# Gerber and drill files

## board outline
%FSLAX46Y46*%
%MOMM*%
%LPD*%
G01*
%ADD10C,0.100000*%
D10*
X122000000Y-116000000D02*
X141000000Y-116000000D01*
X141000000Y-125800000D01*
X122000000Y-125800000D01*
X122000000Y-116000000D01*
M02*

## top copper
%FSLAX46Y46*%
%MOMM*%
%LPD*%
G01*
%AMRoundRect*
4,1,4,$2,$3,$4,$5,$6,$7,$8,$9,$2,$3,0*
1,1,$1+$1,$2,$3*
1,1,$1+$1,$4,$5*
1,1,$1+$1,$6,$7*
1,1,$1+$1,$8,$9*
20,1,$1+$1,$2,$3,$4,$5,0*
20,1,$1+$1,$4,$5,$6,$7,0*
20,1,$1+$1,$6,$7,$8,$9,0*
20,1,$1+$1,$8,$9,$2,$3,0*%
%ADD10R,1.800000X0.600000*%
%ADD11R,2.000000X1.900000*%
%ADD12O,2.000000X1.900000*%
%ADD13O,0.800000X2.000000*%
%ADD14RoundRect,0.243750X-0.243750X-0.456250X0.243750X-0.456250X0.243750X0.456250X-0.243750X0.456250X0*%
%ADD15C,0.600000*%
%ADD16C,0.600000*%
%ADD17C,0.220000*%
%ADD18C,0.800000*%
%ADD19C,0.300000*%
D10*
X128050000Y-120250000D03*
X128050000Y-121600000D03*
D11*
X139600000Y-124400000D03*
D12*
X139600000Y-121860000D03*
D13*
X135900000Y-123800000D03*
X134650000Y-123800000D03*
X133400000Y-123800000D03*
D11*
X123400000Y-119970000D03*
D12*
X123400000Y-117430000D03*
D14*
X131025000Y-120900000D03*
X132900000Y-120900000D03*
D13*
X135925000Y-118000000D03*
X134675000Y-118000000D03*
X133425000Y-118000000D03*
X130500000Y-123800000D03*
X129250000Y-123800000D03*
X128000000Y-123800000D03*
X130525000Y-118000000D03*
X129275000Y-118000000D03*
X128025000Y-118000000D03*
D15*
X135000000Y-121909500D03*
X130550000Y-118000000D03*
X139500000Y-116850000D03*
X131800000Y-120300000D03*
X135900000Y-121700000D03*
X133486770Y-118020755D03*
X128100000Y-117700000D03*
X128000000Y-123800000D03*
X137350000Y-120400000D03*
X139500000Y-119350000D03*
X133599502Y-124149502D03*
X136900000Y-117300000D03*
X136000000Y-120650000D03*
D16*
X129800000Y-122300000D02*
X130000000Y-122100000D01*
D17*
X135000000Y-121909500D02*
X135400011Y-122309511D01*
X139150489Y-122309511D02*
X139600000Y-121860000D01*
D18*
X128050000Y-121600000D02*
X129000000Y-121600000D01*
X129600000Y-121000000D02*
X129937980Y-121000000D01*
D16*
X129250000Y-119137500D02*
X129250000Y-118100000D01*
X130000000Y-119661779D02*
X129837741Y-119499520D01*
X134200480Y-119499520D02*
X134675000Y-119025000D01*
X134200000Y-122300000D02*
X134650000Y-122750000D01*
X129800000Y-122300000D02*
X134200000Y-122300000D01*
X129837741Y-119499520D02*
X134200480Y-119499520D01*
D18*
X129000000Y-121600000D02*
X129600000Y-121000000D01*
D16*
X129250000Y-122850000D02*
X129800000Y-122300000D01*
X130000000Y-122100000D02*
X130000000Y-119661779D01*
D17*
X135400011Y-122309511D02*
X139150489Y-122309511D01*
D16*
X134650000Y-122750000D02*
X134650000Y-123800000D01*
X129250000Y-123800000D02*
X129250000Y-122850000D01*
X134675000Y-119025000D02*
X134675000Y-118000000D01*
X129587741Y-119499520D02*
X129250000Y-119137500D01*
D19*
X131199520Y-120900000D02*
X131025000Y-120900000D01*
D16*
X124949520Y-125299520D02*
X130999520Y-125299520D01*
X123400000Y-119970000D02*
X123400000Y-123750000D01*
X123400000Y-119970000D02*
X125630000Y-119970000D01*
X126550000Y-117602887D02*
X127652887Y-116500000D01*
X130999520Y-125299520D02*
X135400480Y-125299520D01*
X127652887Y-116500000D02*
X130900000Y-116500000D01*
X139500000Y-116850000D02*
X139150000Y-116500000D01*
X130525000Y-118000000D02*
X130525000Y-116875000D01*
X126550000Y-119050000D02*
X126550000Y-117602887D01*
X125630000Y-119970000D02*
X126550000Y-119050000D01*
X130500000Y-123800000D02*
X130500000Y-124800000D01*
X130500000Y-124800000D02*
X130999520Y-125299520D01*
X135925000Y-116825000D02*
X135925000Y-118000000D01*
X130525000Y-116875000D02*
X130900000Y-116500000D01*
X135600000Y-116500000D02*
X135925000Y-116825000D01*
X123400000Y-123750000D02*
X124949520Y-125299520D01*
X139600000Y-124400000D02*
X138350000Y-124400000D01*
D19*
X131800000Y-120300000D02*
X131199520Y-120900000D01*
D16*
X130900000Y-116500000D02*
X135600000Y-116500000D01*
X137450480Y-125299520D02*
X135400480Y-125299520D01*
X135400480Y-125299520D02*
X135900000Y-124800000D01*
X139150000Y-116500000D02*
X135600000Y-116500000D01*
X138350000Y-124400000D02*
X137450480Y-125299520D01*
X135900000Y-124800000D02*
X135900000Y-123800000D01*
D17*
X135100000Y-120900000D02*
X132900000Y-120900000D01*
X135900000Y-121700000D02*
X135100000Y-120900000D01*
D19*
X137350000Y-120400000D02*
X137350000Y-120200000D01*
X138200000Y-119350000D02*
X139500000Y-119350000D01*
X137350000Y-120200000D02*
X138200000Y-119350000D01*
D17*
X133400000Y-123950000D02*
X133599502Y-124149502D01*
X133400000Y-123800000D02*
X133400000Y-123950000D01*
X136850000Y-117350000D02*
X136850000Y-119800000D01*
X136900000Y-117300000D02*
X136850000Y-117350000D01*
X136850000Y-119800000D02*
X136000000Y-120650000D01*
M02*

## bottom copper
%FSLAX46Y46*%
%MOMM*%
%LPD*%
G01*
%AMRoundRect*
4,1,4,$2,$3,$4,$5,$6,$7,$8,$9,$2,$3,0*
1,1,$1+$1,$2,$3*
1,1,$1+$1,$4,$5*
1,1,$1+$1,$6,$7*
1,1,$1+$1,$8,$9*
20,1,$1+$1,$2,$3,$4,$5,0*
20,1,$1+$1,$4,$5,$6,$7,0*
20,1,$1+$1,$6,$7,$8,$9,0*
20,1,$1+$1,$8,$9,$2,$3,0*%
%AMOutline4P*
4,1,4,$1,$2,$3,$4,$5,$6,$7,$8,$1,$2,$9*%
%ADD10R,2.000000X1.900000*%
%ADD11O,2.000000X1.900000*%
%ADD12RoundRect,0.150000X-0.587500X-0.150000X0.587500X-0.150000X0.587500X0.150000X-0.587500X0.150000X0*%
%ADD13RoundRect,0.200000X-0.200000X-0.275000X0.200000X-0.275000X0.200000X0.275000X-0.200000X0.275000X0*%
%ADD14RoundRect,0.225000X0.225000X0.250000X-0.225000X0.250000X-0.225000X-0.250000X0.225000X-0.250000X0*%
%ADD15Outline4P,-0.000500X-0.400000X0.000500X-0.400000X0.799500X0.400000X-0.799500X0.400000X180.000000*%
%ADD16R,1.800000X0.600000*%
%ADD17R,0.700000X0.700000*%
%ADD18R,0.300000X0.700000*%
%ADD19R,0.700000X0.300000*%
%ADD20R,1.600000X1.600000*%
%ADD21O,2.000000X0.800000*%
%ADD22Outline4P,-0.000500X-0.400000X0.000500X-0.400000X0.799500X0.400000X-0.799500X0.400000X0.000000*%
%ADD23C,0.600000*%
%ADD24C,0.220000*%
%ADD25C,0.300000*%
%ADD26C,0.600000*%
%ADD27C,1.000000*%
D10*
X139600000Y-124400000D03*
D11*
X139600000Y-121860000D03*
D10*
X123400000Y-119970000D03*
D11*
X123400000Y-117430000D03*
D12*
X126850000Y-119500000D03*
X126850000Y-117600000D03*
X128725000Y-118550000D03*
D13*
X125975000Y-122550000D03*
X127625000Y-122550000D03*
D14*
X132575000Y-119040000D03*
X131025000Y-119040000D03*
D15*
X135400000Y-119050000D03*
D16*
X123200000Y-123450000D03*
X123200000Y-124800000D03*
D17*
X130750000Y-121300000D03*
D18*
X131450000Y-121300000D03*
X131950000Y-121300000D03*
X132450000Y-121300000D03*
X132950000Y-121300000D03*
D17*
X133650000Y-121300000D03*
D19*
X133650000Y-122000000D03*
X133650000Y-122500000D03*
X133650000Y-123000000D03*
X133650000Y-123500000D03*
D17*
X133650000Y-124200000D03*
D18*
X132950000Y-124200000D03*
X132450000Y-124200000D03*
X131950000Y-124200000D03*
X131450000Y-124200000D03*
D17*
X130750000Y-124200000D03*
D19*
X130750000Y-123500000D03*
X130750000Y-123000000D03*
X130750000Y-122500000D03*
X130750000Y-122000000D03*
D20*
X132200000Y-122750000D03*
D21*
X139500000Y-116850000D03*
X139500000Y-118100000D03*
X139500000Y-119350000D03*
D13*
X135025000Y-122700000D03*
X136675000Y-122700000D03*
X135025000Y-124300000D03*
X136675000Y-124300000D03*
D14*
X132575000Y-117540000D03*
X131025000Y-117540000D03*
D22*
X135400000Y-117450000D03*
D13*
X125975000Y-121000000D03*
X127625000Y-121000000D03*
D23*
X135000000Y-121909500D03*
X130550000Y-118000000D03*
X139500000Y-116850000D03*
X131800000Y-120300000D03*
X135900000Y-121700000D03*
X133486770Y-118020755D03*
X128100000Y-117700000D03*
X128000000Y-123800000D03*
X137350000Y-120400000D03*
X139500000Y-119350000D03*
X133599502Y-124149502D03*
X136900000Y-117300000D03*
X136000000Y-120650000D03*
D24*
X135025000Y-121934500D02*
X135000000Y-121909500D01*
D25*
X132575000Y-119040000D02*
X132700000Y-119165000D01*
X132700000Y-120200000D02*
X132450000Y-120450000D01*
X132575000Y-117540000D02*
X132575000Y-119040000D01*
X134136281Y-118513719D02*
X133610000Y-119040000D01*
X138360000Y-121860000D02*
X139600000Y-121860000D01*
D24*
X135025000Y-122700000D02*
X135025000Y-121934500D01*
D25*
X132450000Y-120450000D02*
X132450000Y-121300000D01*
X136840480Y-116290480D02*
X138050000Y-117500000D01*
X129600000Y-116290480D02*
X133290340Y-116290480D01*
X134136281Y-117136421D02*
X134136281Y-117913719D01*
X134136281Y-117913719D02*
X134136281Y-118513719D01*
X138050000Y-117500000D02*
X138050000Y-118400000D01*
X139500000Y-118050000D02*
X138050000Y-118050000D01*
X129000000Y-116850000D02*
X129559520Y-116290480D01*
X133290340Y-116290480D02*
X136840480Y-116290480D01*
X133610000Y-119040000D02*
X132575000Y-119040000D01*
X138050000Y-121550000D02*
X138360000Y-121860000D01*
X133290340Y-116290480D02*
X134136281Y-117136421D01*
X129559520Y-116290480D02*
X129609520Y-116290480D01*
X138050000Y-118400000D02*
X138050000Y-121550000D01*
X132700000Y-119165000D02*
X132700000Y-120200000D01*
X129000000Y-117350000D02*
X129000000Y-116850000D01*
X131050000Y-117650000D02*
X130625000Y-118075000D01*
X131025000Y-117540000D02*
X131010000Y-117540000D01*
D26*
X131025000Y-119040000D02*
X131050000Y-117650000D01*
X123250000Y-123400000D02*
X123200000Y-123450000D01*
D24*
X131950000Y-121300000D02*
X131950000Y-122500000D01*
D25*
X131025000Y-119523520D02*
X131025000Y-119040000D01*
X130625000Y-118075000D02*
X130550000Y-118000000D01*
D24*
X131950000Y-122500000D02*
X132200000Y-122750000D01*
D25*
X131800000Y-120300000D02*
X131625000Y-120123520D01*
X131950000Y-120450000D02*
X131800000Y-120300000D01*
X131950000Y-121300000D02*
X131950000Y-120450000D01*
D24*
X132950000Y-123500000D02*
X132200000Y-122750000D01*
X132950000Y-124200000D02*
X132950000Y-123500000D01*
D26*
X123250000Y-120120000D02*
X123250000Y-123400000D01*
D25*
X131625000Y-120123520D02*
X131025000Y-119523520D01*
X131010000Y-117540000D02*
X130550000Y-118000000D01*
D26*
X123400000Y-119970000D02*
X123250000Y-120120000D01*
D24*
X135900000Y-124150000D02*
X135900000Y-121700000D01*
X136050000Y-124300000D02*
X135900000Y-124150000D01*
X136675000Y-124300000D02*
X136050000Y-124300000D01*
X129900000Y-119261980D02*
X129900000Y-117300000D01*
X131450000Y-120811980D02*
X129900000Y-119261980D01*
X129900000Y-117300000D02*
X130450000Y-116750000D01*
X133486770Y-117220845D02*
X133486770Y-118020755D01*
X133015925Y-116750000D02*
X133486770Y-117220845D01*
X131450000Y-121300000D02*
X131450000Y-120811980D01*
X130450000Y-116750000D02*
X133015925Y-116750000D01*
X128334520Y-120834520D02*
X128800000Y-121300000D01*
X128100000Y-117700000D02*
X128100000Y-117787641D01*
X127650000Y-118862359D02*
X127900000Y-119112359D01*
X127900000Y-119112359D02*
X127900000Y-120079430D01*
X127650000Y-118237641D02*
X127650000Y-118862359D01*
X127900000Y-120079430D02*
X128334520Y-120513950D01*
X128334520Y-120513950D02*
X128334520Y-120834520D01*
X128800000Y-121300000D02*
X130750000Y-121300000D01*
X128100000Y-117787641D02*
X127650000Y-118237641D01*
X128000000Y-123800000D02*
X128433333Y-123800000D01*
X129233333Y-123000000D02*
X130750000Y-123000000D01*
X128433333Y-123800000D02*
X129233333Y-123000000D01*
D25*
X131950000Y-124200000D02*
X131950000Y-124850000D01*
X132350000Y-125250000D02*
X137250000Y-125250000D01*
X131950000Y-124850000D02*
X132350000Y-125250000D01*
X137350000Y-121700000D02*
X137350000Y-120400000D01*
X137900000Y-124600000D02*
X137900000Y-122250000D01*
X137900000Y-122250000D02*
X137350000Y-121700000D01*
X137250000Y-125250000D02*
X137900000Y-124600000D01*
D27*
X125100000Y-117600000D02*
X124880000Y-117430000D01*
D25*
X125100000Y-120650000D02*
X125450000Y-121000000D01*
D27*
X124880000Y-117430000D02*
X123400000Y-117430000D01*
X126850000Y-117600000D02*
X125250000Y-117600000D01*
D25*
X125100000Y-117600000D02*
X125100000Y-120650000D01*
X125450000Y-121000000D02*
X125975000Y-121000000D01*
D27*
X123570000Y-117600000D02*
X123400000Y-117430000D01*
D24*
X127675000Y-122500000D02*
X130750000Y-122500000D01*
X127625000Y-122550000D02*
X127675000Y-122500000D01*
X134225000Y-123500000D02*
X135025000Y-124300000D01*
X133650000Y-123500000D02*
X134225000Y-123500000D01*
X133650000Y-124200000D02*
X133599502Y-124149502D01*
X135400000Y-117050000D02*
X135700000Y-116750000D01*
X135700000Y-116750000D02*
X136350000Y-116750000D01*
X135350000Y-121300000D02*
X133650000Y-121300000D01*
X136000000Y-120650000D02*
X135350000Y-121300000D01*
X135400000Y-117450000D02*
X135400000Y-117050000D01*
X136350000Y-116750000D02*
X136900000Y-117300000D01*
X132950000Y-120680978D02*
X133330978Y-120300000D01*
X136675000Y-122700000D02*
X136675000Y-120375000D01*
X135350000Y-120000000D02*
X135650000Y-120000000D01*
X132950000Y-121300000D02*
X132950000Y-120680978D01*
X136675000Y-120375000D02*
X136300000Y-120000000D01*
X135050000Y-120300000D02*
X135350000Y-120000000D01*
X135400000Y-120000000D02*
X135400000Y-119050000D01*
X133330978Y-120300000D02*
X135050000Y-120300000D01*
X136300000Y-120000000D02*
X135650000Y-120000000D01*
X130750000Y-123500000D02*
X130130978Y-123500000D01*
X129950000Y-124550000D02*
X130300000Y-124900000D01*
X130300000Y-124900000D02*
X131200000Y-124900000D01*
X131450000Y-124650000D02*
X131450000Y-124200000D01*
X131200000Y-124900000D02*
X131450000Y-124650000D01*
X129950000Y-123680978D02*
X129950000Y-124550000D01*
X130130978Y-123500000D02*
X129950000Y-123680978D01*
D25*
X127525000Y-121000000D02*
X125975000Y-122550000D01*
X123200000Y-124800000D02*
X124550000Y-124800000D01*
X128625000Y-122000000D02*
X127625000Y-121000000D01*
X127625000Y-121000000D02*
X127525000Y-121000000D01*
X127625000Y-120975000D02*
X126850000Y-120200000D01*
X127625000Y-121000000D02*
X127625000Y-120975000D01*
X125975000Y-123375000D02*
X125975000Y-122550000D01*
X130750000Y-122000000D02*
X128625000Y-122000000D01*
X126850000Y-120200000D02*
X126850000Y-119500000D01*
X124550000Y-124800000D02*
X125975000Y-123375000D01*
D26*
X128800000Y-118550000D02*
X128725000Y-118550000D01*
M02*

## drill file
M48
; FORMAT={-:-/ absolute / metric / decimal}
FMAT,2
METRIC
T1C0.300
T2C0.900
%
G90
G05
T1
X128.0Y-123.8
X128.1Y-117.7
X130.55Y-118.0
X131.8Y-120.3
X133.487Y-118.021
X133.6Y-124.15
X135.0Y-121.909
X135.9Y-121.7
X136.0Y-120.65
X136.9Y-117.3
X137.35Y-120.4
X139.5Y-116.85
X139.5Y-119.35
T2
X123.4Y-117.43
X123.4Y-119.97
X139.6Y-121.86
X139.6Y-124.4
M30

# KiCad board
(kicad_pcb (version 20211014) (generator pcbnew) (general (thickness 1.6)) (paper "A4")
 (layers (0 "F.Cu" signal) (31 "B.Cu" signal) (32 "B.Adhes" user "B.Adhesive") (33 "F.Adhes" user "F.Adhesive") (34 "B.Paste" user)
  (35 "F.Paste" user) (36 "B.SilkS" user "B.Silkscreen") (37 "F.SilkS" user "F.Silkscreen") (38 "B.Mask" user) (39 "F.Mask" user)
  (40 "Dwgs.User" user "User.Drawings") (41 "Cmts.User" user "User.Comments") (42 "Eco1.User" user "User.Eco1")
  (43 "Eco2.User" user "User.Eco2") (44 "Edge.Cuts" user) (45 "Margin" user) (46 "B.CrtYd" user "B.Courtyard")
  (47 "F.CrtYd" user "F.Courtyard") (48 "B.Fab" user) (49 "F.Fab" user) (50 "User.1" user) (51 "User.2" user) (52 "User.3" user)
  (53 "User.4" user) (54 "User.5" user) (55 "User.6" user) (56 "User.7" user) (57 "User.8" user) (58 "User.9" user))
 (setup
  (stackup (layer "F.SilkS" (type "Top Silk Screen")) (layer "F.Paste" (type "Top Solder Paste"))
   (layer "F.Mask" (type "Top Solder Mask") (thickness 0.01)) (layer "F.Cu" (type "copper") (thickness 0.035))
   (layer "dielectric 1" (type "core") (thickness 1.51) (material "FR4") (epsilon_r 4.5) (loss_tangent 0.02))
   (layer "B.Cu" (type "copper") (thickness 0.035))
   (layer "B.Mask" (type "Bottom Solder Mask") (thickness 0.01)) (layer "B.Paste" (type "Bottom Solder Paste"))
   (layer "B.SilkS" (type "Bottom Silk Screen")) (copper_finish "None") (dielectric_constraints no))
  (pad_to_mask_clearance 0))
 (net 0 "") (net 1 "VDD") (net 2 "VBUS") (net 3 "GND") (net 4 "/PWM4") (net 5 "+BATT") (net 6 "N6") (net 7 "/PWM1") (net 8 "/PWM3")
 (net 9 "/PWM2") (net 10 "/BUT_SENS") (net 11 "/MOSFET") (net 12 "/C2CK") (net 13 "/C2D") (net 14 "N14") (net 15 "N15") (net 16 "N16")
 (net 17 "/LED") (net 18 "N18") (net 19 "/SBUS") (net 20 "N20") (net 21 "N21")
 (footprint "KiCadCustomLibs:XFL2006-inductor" (layer "F.Cu") (at 128.05 120.925 -90)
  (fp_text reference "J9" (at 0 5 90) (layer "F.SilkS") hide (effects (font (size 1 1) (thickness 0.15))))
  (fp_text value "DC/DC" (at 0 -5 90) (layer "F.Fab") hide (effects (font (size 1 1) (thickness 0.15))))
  (pad "1" smd rect locked (at -0.675 0 270) (size 0.6 1.8) (layers "F.Cu" "F.Paste" "F.Mask") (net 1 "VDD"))
  (pad "2" smd rect locked (at 0.675 0 270) (size 0.6 1.8) (layers "F.Cu" "F.Paste" "F.Mask") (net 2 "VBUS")))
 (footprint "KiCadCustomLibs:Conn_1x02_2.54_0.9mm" (layer "F.Cu") (at 139.6 124.4 180)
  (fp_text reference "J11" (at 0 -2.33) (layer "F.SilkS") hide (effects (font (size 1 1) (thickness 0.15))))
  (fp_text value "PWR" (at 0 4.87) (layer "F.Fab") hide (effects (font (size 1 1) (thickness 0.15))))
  (pad "1" thru_hole rect locked (at 0 0 180) (size 2 1.9) (drill 0.9) (layers *.Cu *.Mask) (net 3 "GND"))
  (pad "2" thru_hole oval locked (at 0 2.54 180) (size 2 1.9) (drill 0.9) (layers *.Cu *.Mask) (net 2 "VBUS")))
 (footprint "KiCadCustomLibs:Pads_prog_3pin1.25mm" (layer "F.Cu") (at 134.675 123.8 180)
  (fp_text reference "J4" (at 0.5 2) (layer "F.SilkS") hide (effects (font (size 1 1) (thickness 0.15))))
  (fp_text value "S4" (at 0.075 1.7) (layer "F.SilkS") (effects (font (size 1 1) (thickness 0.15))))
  (pad "1" smd oval locked (at -1.225 0 180) (size 0.8 2) (layers "F.Cu" "F.Paste" "F.Mask") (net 3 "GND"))
  (pad "2" smd oval locked (at 0.025 0 180) (size 0.8 2) (layers "F.Cu" "F.Paste" "F.Mask") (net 2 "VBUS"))
  (pad "3" smd oval locked (at 1.275 0 180) (size 0.8 2) (layers "F.Cu" "F.Paste" "F.Mask") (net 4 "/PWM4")))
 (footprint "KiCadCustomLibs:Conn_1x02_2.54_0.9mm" (layer "F.Cu") (at 123.4 119.97 180)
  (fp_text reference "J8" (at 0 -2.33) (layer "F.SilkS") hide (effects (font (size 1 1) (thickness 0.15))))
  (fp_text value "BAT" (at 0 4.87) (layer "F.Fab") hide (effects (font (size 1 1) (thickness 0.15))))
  (pad "1" thru_hole rect locked (at 0 0 180) (size 2 1.9) (drill 0.9) (layers *.Cu *.Mask) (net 3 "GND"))
  (pad "2" thru_hole oval locked (at 0 2.54 180) (size 2 1.9) (drill 0.9) (layers *.Cu *.Mask) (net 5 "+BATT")))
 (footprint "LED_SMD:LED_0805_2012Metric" (layer "F.Cu") (at 131.9625 120.9)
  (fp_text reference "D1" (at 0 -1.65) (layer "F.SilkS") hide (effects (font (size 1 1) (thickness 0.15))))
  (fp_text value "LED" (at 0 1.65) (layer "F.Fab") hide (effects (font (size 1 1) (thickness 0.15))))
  (pad "1" smd roundrect (at -0.9375 0) (size 0.975 1.4) (layers "F.Cu" "F.Paste" "F.Mask") (roundrect_rratio 0.25) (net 3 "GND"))
  (pad "2" smd roundrect (at 0.9375 0) (size 0.975 1.4) (layers "F.Cu" "F.Paste" "F.Mask") (roundrect_rratio 0.25) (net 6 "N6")))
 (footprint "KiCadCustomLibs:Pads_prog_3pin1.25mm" (layer "F.Cu") (at 134.7 118 180)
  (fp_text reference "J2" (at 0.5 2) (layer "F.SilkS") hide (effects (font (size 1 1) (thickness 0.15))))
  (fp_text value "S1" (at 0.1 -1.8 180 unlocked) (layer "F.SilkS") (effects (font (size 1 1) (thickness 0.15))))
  (pad "1" smd oval locked (at -1.225 0 180) (size 0.8 2) (layers "F.Cu" "F.Paste" "F.Mask") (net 3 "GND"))
  (pad "2" smd oval locked (at 0.025 0 180) (size 0.8 2) (layers "F.Cu" "F.Paste" "F.Mask") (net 2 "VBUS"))
  (pad "3" smd oval locked (at 1.275 0 180) (size 0.8 2) (layers "F.Cu" "F.Paste" "F.Mask") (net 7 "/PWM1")))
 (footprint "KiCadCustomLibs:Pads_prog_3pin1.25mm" (layer "F.Cu") (at 129.275 123.8 180)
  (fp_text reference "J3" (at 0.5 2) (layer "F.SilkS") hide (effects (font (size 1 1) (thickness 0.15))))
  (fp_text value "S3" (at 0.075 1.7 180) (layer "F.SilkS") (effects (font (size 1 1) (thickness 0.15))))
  (pad "1" smd oval locked (at -1.225 0 180) (size 0.8 2) (layers "F.Cu" "F.Paste" "F.Mask") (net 3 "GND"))
  (pad "2" smd oval locked (at 0.025 0 180) (size 0.8 2) (layers "F.Cu" "F.Paste" "F.Mask") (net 2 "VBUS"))
  (pad "3" smd oval locked (at 1.275 0 180) (size 0.8 2) (layers "F.Cu" "F.Paste" "F.Mask") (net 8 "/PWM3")))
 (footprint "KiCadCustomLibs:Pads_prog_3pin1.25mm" (layer "F.Cu") (at 129.3 118 180)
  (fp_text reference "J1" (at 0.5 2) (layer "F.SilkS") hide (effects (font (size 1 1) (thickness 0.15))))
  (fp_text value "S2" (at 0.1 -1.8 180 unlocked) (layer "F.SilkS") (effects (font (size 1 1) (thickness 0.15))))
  (pad "1" smd oval locked (at -1.225 0 180) (size 0.8 2) (layers "F.Cu" "F.Paste" "F.Mask") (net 3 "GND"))
  (pad "2" smd oval locked (at 0.025 0 180) (size 0.8 2) (layers "F.Cu" "F.Paste" "F.Mask") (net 2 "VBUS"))
  (pad "3" smd oval locked (at 1.275 0 180) (size 0.8 2) (layers "F.Cu" "F.Paste" "F.Mask") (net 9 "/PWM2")))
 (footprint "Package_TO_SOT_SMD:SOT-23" (layer "B.Cu") (at 127.7875 118.55)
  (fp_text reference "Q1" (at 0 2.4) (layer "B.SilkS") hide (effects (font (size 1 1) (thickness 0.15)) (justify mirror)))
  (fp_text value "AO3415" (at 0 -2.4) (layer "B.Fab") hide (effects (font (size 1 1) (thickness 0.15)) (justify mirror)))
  (pad "1" smd roundrect (at -0.9375 0.95) (size 1.475 0.6) (layers "B.Cu" "B.Paste" "B.Mask") (roundrect_rratio 0.25) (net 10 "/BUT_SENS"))
  (pad "2" smd roundrect (at -0.9375 -0.95) (size 1.475 0.6) (layers "B.Cu" "B.Paste" "B.Mask") (roundrect_rratio 0.25) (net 5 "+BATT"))
  (pad "3" smd roundrect (at 0.9375 0) (size 1.475 0.6) (layers "B.Cu" "B.Paste" "B.Mask") (roundrect_rratio 0.25) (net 1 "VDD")))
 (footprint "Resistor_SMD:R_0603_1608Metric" (layer "B.Cu") (at 126.8 122.55)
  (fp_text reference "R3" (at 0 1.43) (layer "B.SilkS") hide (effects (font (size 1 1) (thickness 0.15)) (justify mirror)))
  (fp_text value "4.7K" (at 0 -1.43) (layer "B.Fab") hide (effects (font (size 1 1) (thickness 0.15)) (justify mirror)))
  (pad "1" smd roundrect (at -0.825 0) (size 0.8 0.95) (layers "B.Cu" "B.Paste" "B.Mask") (roundrect_rratio 0.25) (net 10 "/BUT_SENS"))
  (pad "2" smd roundrect (at 0.825 0) (size 0.8 0.95) (layers "B.Cu" "B.Paste" "B.Mask") (roundrect_rratio 0.25) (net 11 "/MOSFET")))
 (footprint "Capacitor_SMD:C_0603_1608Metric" (layer "B.Cu") (at 131.8 119.04 180)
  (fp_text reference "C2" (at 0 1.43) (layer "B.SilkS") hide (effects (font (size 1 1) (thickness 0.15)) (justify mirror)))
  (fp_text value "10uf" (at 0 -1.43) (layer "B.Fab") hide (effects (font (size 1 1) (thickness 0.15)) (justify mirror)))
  (pad "1" smd roundrect (at -0.775 0 180) (size 0.9 0.95) (layers "B.Cu" "B.Paste" "B.Mask") (roundrect_rratio 0.25) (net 2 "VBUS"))
  (pad "2" smd roundrect (at 0.775 0 180) (size 0.9 0.95) (layers "B.Cu" "B.Paste" "B.Mask") (roundrect_rratio 0.25) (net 3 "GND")))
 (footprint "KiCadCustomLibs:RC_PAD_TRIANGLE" (layer "B.Cu") (at 135.4 119.05 180)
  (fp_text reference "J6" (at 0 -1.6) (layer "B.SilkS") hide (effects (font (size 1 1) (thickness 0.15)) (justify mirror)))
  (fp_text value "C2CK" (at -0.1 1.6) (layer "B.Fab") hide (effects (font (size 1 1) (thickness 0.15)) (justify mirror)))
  (pad "1" smd trapezoid locked (at 0 0 180) (size 0.8 0.8) (rect_delta 0 -0.799) (layers "B.Cu" "B.Paste" "B.Mask") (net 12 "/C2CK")))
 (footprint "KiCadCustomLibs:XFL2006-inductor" (layer "B.Cu") (at 123.2 124.125 -90)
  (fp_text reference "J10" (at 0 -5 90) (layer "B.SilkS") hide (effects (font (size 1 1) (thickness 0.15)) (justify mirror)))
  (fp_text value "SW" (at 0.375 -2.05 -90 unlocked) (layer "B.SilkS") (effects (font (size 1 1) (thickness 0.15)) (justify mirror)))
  (pad "1" smd rect locked (at -0.675 0 270) (size 0.6 1.8) (layers "B.Cu" "B.Paste" "B.Mask") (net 3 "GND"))
  (pad "2" smd rect locked (at 0.675 0 270) (size 0.6 1.8) (layers "B.Cu" "B.Paste" "B.Mask") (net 10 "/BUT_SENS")))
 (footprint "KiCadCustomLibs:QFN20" (layer "B.Cu") (at 132.2 122.75)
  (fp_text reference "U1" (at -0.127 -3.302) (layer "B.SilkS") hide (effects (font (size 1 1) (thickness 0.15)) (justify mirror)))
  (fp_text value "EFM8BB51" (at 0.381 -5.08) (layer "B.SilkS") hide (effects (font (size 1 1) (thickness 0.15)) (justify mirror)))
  (pad "1" smd rect locked (at -1.45 -1.45) (size 0.7 0.7) (layers "B.Cu" "B.Paste" "B.Mask") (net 9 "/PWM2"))
  (pad "2" smd rect locked (at -0.75 -1.45) (size 0.3 0.7) (layers "B.Cu" "B.Paste" "B.Mask") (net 7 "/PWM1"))
  (pad "3" smd rect locked (at -0.25 -1.45) (size 0.3 0.7) (layers "B.Cu" "B.Paste" "B.Mask") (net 3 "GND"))
  (pad "4" smd rect locked (at 0.25 -1.45) (size 0.3 0.7) (layers "B.Cu" "B.Paste" "B.Mask") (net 2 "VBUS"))
  (pad "5" smd rect locked (at 0.75 -1.45) (size 0.3 0.7) (layers "B.Cu" "B.Paste" "B.Mask") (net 12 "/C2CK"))
  (pad "6" smd rect locked (at 1.45 -1.45) (size 0.7 0.7) (layers "B.Cu" "B.Paste" "B.Mask") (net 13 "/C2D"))
  (pad "7" smd rect locked (at 1.45 -0.75 270) (size 0.3 0.7) (layers "B.Cu" "B.Paste" "B.Mask") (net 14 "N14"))
  (pad "8" smd rect locked (at 1.45 -0.25 270) (size 0.3 0.7) (layers "B.Cu" "B.Paste" "B.Mask") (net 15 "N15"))
  (pad "9" smd rect locked (at 1.45 0.25 270) (size 0.3 0.7) (layers "B.Cu" "B.Paste" "B.Mask") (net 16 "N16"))
  (pad "10" smd rect locked (at 1.45 0.75 270) (size 0.3 0.7) (layers "B.Cu" "B.Paste" "B.Mask") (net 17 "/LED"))
  (pad "11" smd rect locked (at 1.45 1.45) (size 0.7 0.7) (layers "B.Cu" "B.Paste" "B.Mask") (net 4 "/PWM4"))
  (pad "12" smd rect locked (at 0.75 1.45) (size 0.3 0.7) (layers "B.Cu" "B.Paste" "B.Mask") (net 3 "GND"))
  (pad "13" smd rect locked (at 0.25 1.45) (size 0.3 0.7) (layers "B.Cu" "B.Paste" "B.Mask") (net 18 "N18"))
  (pad "14" smd rect locked (at -0.25 1.45) (size 0.3 0.7) (layers "B.Cu" "B.Paste" "B.Mask") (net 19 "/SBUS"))
  (pad "15" smd rect locked (at -0.75 1.45) (size 0.3 0.7) (layers "B.Cu" "B.Paste" "B.Mask") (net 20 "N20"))
  (pad "16" smd rect locked (at -1.45 1.45) (size 0.7 0.7) (layers "B.Cu" "B.Paste" "B.Mask") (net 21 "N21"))
  (pad "17" smd rect locked (at -1.45 0.75 270) (size 0.3 0.7) (layers "B.Cu" "B.Paste" "B.Mask") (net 20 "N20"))
  (pad "18" smd rect locked (at -1.45 0.25 270) (size 0.3 0.7) (layers "B.Cu" "B.Paste" "B.Mask") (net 8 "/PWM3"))
  (pad "19" smd rect locked (at -1.45 -0.25 270) (size 0.3 0.7) (layers "B.Cu" "B.Paste" "B.Mask") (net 11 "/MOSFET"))
  (pad "20" smd rect locked (at -1.45 -0.75 270) (size 0.3 0.7) (layers "B.Cu" "B.Paste" "B.Mask") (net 10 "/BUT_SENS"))
  (pad "21" smd rect locked (at 0 0) (size 1.6 1.6) (layers "B.Cu" "B.Paste" "B.Mask") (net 3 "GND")))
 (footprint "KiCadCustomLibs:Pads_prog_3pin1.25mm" (layer "B.Cu") (at 139.5 118.075 -90)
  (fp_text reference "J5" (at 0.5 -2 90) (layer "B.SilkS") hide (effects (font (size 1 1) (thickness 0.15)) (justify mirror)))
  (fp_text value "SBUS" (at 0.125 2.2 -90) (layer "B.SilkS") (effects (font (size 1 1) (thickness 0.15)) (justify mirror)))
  (pad "1" smd oval locked (at -1.225 0 270) (size 0.8 2) (layers "B.Cu" "B.Paste" "B.Mask") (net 3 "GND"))
  (pad "2" smd oval locked (at 0.025 0 270) (size 0.8 2) (layers "B.Cu" "B.Paste" "B.Mask") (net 2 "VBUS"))
  (pad "3" smd oval locked (at 1.275 0 270) (size 0.8 2) (layers "B.Cu" "B.Paste" "B.Mask") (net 19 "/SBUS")))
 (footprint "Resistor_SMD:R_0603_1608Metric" (layer "B.Cu") (at 135.85 122.7)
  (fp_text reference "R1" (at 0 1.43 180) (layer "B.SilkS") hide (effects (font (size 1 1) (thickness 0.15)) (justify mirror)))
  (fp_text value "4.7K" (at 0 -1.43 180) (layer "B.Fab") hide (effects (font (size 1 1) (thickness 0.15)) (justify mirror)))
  (pad "1" smd roundrect (at -0.825 0) (size 0.8 0.95) (layers "B.Cu" "B.Paste" "B.Mask") (roundrect_rratio 0.25) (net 2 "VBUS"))
  (pad "2" smd roundrect (at 0.825 0) (size 0.8 0.95) (layers "B.Cu" "B.Paste" "B.Mask") (roundrect_rratio 0.25) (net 12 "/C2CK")))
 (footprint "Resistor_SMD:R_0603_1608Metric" (layer "B.Cu") (at 135.85 124.3)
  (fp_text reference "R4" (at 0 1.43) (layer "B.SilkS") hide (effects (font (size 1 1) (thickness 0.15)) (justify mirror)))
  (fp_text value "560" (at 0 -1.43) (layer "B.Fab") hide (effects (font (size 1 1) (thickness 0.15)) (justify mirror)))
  (pad "1" smd roundrect (at -0.825 0) (size 0.8 0.95) (layers "B.Cu" "B.Paste" "B.Mask") (roundrect_rratio 0.25) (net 17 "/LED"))
  (pad "2" smd roundrect (at 0.825 0) (size 0.8 0.95) (layers "B.Cu" "B.Paste" "B.Mask") (roundrect_rratio 0.25) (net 6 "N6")))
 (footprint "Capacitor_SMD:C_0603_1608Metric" (layer "B.Cu") (at 131.8 117.54 180)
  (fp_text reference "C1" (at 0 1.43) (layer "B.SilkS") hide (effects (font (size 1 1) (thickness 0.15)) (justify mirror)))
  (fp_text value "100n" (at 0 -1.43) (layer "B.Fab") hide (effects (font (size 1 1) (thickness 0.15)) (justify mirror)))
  (pad "1" smd roundrect (at -0.775 0 180) (size 0.9 0.95) (layers "B.Cu" "B.Paste" "B.Mask") (roundrect_rratio 0.25) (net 2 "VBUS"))
  (pad "2" smd roundrect (at 0.775 0 180) (size 0.9 0.95) (layers "B.Cu" "B.Paste" "B.Mask") (roundrect_rratio 0.25) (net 3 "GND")))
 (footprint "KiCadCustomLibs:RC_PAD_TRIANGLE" (layer "B.Cu") (at 135.4 117.45)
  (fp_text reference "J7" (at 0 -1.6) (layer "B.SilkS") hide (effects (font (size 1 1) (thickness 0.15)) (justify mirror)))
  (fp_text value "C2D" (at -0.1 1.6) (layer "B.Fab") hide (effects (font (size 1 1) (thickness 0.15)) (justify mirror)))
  (pad "1" smd trapezoid locked (at 0 0) (size 0.8 0.8) (rect_delta 0 -0.799) (layers "B.Cu" "B.Paste" "B.Mask") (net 13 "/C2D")))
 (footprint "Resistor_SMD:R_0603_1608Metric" (layer "B.Cu") (at 126.8 121)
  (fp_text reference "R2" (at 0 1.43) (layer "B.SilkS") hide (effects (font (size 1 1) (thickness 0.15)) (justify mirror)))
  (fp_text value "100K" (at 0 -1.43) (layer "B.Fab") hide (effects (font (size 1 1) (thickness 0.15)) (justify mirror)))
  (pad "1" smd roundrect (at -0.825 0) (size 0.8 0.95) (layers "B.Cu" "B.Paste" "B.Mask") (roundrect_rratio 0.25) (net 5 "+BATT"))
  (pad "2" smd roundrect (at 0.825 0) (size 0.8 0.95) (layers "B.Cu" "B.Paste" "B.Mask") (roundrect_rratio 0.25) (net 10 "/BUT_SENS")))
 (gr_rect (start 122 116) (end 141 125.8) (layer "Edge.Cuts") (width 0.1) (fill none))
 (segment (start 129.8 122.3) (end 130 122.1) (width 0.6) (layer "F.Cu") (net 2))
 (segment (start 135 121.9095) (end 135.400011 122.309511) (width 0.22) (layer "F.Cu") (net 2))
 (segment (start 139.150489 122.309511) (end 139.6 121.86) (width 0.22) (layer "F.Cu") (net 2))
 (segment (start 128.05 121.6) (end 129 121.6) (width 0.8) (layer "F.Cu") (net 2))
 (segment (start 129.6 121) (end 129.93798 121) (width 0.8) (layer "F.Cu") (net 2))
 (segment (start 129.25 119.1375) (end 129.25 118.1) (width 0.6) (layer "F.Cu") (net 2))
 (segment (start 130 119.661779) (end 129.837741 119.49952) (width 0.6) (layer "F.Cu") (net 2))
 (segment (start 134.20048 119.49952) (end 134.675 119.025) (width 0.6) (layer "F.Cu") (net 2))
 (segment (start 134.2 122.3) (end 134.65 122.75) (width 0.6) (layer "F.Cu") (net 2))
 (segment (start 129.8 122.3) (end 134.2 122.3) (width 0.6) (layer "F.Cu") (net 2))
 (segment (start 129.837741 119.49952) (end 134.20048 119.49952) (width 0.6) (layer "F.Cu") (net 2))
 (segment (start 129 121.6) (end 129.6 121) (width 0.8) (layer "F.Cu") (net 2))
 (segment (start 129.25 122.85) (end 129.8 122.3) (width 0.6) (layer "F.Cu") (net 2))
 (segment (start 130 122.1) (end 130 119.661779) (width 0.6) (layer "F.Cu") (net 2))
 (segment (start 135.400011 122.309511) (end 139.150489 122.309511) (width 0.22) (layer "F.Cu") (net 2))
 (segment (start 134.65 122.75) (end 134.65 123.8) (width 0.6) (layer "F.Cu") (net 2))
 (segment (start 129.25 123.8) (end 129.25 122.85) (width 0.6) (layer "F.Cu") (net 2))
 (segment (start 134.675 119.025) (end 134.675 118) (width 0.6) (layer "F.Cu") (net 2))
 (segment (start 129.587741 119.49952) (end 129.25 119.1375) (width 0.6) (layer "F.Cu") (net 2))
 (via (at 135 121.9095) (size 0.6) (drill 0.3) (layers "F.Cu" "B.Cu") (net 2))
 (segment (start 135.025 121.9345) (end 135 121.9095) (width 0.22) (layer "B.Cu") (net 2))
 (segment (start 132.575 119.04) (end 132.7 119.165) (width 0.3) (layer "B.Cu") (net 2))
 (segment (start 132.7 120.2) (end 132.45 120.45) (width 0.3) (layer "B.Cu") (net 2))
 (segment (start 132.575 117.54) (end 132.575 119.04) (width 0.3) (layer "B.Cu") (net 2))
 (segment (start 134.136281 118.513719) (end 133.61 119.04) (width 0.3) (layer "B.Cu") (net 2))
 (segment (start 138.36 121.86) (end 139.6 121.86) (width 0.3) (layer "B.Cu") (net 2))
 (segment (start 135.025 122.7) (end 135.025 121.9345) (width 0.22) (layer "B.Cu") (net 2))
 (segment (start 132.45 120.45) (end 132.45 121.3) (width 0.3) (layer "B.Cu") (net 2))
 (segment (start 136.84048 116.29048) (end 138.05 117.5) (width 0.3) (layer "B.Cu") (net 2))
 (segment (start 129.6 116.29048) (end 133.29034 116.29048) (width 0.3) (layer "B.Cu") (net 2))
 (segment (start 134.136281 117.136421) (end 134.136281 117.913719) (width 0.3) (layer "B.Cu") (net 2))
 (segment (start 134.136281 117.913719) (end 134.136281 118.513719) (width 0.3) (layer "B.Cu") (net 2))
 (segment (start 138.05 117.5) (end 138.05 118.4) (width 0.3) (layer "B.Cu") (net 2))
 (segment (start 139.5 118.05) (end 138.05 118.05) (width 0.3) (layer "B.Cu") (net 2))
 (segment (start 129 116.85) (end 129.55952 116.29048) (width 0.3) (layer "B.Cu") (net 2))
 (segment (start 133.29034 116.29048) (end 136.84048 116.29048) (width 0.3) (layer "B.Cu") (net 2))
 (segment (start 133.61 119.04) (end 132.575 119.04) (width 0.3) (layer "B.Cu") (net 2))
 (segment (start 138.05 121.55) (end 138.36 121.86) (width 0.3) (layer "B.Cu") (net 2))
 (segment (start 133.29034 116.29048) (end 134.136281 117.136421) (width 0.3) (layer "B.Cu") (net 2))
 (segment (start 129.55952 116.29048) (end 129.60952 116.29048) (width 0.3) (layer "B.Cu") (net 2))
 (segment (start 138.05 118.4) (end 138.05 121.55) (width 0.3) (layer "B.Cu") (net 2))
 (segment (start 132.7 119.165) (end 132.7 120.2) (width 0.3) (layer "B.Cu") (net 2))
 (segment (start 129 117.35) (end 129 116.85) (width 0.3) (layer "B.Cu") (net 2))
 (segment (start 131.19952 120.9) (end 131.025 120.9) (width 0.3) (layer "F.Cu") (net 3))
 (segment (start 124.94952 125.29952) (end 130.99952 125.29952) (width 0.6) (layer "F.Cu") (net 3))
 (segment (start 123.4 119.97) (end 123.4 123.75) (width 0.6) (layer "F.Cu") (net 3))
 (segment (start 123.4 119.97) (end 125.63 119.97) (width 0.6) (layer "F.Cu") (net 3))
 (segment (start 126.55 117.602887) (end 127.652887 116.5) (width 0.6) (layer "F.Cu") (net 3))
 (segment (start 130.99952 125.29952) (end 135.40048 125.29952) (width 0.6) (layer "F.Cu") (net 3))
 (segment (start 127.652887 116.5) (end 130.9 116.5) (width 0.6) (layer "F.Cu") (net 3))
 (segment (start 139.5 116.85) (end 139.15 116.5) (width 0.6) (layer "F.Cu") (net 3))
 (segment (start 130.525 118) (end 130.525 116.875) (width 0.6) (layer "F.Cu") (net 3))
 (segment (start 126.55 119.05) (end 126.55 117.602887) (width 0.6) (layer "F.Cu") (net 3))
 (segment (start 125.63 119.97) (end 126.55 119.05) (width 0.6) (layer "F.Cu") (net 3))
 (segment (start 130.5 123.8) (end 130.5 124.8) (width 0.6) (layer "F.Cu") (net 3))
 (segment (start 130.5 124.8) (end 130.99952 125.29952) (width 0.6) (layer "F.Cu") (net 3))
 (segment (start 135.925 116.825) (end 135.925 118) (width 0.6) (layer "F.Cu") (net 3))
 (segment (start 130.525 116.875) (end 130.9 116.5) (width 0.6) (layer "F.Cu") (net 3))
 (segment (start 135.6 116.5) (end 135.925 116.825) (width 0.6) (layer "F.Cu") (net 3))
 (segment (start 123.4 123.75) (end 124.94952 125.29952) (width 0.6) (layer "F.Cu") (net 3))
 (segment (start 139.6 124.4) (end 138.35 124.4) (width 0.6) (layer "F.Cu") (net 3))
 (segment (start 131.8 120.3) (end 131.19952 120.9) (width 0.3) (layer "F.Cu") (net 3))
 (segment (start 130.9 116.5) (end 135.6 116.5) (width 0.6) (layer "F.Cu") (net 3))
 (segment (start 137.45048 125.29952) (end 135.40048 125.29952) (width 0.6) (layer "F.Cu") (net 3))
 (segment (start 135.40048 125.29952) (end 135.9 124.8) (width 0.6) (layer "F.Cu") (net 3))
 (segment (start 139.15 116.5) (end 135.6 116.5) (width 0.6) (layer "F.Cu") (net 3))
 (segment (start 138.35 124.4) (end 137.45048 125.29952) (width 0.6) (layer "F.Cu") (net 3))
 (segment (start 135.9 124.8) (end 135.9 123.8) (width 0.6) (layer "F.Cu") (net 3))
 (via (at 130.55 118) (size 0.6) (drill 0.3) (layers "F.Cu" "B.Cu") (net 3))
 (via (at 139.5 116.85) (size 0.6) (drill 0.3) (layers "F.Cu" "B.Cu") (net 3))
 (via (at 131.8 120.3) (size 0.6) (drill 0.3) (layers "F.Cu" "B.Cu") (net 3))
 (segment (start 131.05 117.65) (end 130.625 118.075) (width 0.3) (layer "B.Cu") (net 3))
 (segment (start 131.025 117.54) (end 131.01 117.54) (width 0.3) (layer "B.Cu") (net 3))
 (segment (start 131.025 119.04) (end 131.05 117.65) (width 0.6) (layer "B.Cu") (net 3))
 (segment (start 123.25 123.4) (end 123.2 123.45) (width 0.6) (layer "B.Cu") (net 3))
 (segment (start 131.95 121.3) (end 131.95 122.5) (width 0.22) (layer "B.Cu") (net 3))
 (segment (start 131.025 119.52352) (end 131.025 119.04) (width 0.3) (layer "B.Cu") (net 3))
 (segment (start 130.625 118.075) (end 130.55 118) (width 0.3) (layer "B.Cu") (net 3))
 (segment (start 131.95 122.5) (end 132.2 122.75) (width 0.22) (layer "B.Cu") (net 3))
 (segment (start 131.8 120.3) (end 131.625 120.12352) (width 0.3) (layer "B.Cu") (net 3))
 (segment (start 131.95 120.45) (end 131.8 120.3) (width 0.3) (layer "B.Cu") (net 3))
 (segment (start 131.95 121.3) (end 131.95 120.45) (width 0.3) (layer "B.Cu") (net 3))
 (segment (start 132.95 123.5) (end 132.2 122.75) (width 0.22) (layer "B.Cu") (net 3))
 (segment (start 132.95 124.2) (end 132.95 123.5) (width 0.22) (layer "B.Cu") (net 3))
 (segment (start 123.25 120.12) (end 123.25 123.4) (width 0.6) (layer "B.Cu") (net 3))
 (segment (start 131.625 120.12352) (end 131.025 119.52352) (width 0.3) (layer "B.Cu") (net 3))
 (segment (start 131.01 117.54) (end 130.55 118) (width 0.3) (layer "B.Cu") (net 3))
 (segment (start 123.4 119.97) (end 123.25 120.12) (width 0.6) (layer "B.Cu") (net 3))
 (segment (start 135.1 120.9) (end 132.9 120.9) (width 0.22) (layer "F.Cu") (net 6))
 (segment (start 135.9 121.7) (end 135.1 120.9) (width 0.22) (layer "F.Cu") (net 6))
 (via (at 135.9 121.7) (size 0.6) (drill 0.3) (layers "F.Cu" "B.Cu") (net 6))
 (segment (start 135.9 124.15) (end 135.9 121.7) (width 0.22) (layer "B.Cu") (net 6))
 (segment (start 136.05 124.3) (end 135.9 124.15) (width 0.22) (layer "B.Cu") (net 6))
 (segment (start 136.675 124.3) (end 136.05 124.3) (width 0.22) (layer "B.Cu") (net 6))
 (via (at 133.48677 118.020755) (size 0.6) (drill 0.3) (layers "F.Cu" "B.Cu") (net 7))
 (segment (start 129.9 119.26198) (end 129.9 117.3) (width 0.22) (layer "B.Cu") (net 7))
 (segment (start 131.45 120.81198) (end 129.9 119.26198) (width 0.22) (layer "B.Cu") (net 7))
 (segment (start 129.9 117.3) (end 130.45 116.75) (width 0.22) (layer "B.Cu") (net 7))
 (segment (start 133.48677 117.220845) (end 133.48677 118.020755) (width 0.22) (layer "B.Cu") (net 7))
 (segment (start 133.015925 116.75) (end 133.48677 117.220845) (width 0.22) (layer "B.Cu") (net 7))
 (segment (start 131.45 121.3) (end 131.45 120.81198) (width 0.22) (layer "B.Cu") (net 7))
 (segment (start 130.45 116.75) (end 133.015925 116.75) (width 0.22) (layer "B.Cu") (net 7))
 (via (at 128.1 117.7) (size 0.6) (drill 0.3) (layers "F.Cu" "B.Cu") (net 9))
 (segment (start 128.33452 120.83452) (end 128.8 121.3) (width 0.22) (layer "B.Cu") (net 9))
 (segment (start 128.1 117.7) (end 128.1 117.787641) (width 0.22) (layer "B.Cu") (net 9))
 (segment (start 127.65 118.862359) (end 127.9 119.112359) (width 0.22) (layer "B.Cu") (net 9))
 (segment (start 127.9 119.112359) (end 127.9 120.07943) (width 0.22) (layer "B.Cu") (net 9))
 (segment (start 127.65 118.237641) (end 127.65 118.862359) (width 0.22) (layer "B.Cu") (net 9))
 (segment (start 127.9 120.07943) (end 128.33452 120.51395) (width 0.22) (layer "B.Cu") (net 9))
 (segment (start 128.33452 120.51395) (end 128.33452 120.83452) (width 0.22) (layer "B.Cu") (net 9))
 (segment (start 128.8 121.3) (end 130.75 121.3) (width 0.22) (layer "B.Cu") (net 9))
 (segment (start 128.1 117.787641) (end 127.65 118.237641) (width 0.22) (layer "B.Cu") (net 9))
 (via (at 128 123.8) (size 0.6) (drill 0.3) (layers "F.Cu" "B.Cu") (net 8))
 (segment (start 128 123.8) (end 128.433333 123.8) (width 0.22) (layer "B.Cu") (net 8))
 (segment (start 129.233333 123) (end 130.75 123) (width 0.22) (layer "B.Cu") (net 8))
 (segment (start 128.433333 123.8) (end 129.233333 123) (width 0.22) (layer "B.Cu") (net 8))
 (segment (start 137.35 120.4) (end 137.35 120.2) (width 0.3) (layer "F.Cu") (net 19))
 (segment (start 138.2 119.35) (end 139.5 119.35) (width 0.3) (layer "F.Cu") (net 19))
 (segment (start 137.35 120.2) (end 138.2 119.35) (width 0.3) (layer "F.Cu") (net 19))
 (via (at 137.35 120.4) (size 0.6) (drill 0.3) (layers "F.Cu" "B.Cu") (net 19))
 (via (at 139.5 119.35) (size 0.6) (drill 0.3) (layers "F.Cu" "B.Cu") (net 19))
 (segment (start 131.95 124.2) (end 131.95 124.85) (width 0.3) (layer "B.Cu") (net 19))
 (segment (start 132.35 125.25) (end 137.25 125.25) (width 0.3) (layer "B.Cu") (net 19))
 (segment (start 131.95 124.85) (end 132.35 125.25) (width 0.3) (layer "B.Cu") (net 19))
 (segment (start 137.35 121.7) (end 137.35 120.4) (width 0.3) (layer "B.Cu") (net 19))
 (segment (start 137.9 124.6) (end 137.9 122.25) (width 0.3) (layer "B.Cu") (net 19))
 (segment (start 137.9 122.25) (end 137.35 121.7) (width 0.3) (layer "B.Cu") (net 19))
 (segment (start 137.25 125.25) (end 137.9 124.6) (width 0.3) (layer "B.Cu") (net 19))
 (segment (start 125.1 117.6) (end 124.88 117.43) (width 1) (layer "B.Cu") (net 5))
 (segment (start 125.1 120.65) (end 125.45 121) (width 0.3) (layer "B.Cu") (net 5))
 (segment (start 124.88 117.43) (end 123.4 117.43) (width 1) (layer "B.Cu") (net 5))
 (segment (start 126.85 117.6) (end 125.25 117.6) (width 1) (layer "B.Cu") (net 5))
 (segment (start 125.1 117.6) (end 125.1 120.65) (width 0.3) (layer "B.Cu") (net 5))
 (segment (start 125.45 121) (end 125.975 121) (width 0.3) (layer "B.Cu") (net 5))
 (segment (start 123.57 117.6) (end 123.4 117.43) (width 1) (layer "B.Cu") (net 5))
 (segment (start 127.675 122.5) (end 130.75 122.5) (width 0.22) (layer "B.Cu") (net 11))
 (segment (start 127.625 122.55) (end 127.675 122.5) (width 0.22) (layer "B.Cu") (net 11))
 (segment (start 134.225 123.5) (end 135.025 124.3) (width 0.22) (layer "B.Cu") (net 17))
 (segment (start 133.65 123.5) (end 134.225 123.5) (width 0.22) (layer "B.Cu") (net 17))
 (segment (start 133.4 123.95) (end 133.599502 124.149502) (width 0.22) (layer "F.Cu") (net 4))
 (segment (start 133.4 123.8) (end 133.4 123.95) (width 0.22) (layer "F.Cu") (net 4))
 (via (at 133.599502 124.149502) (size 0.6) (drill 0.3) (layers "F.Cu" "B.Cu") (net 4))
 (segment (start 133.65 124.2) (end 133.599502 124.149502) (width 0.22) (layer "B.Cu") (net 4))
 (segment (start 136.85 117.35) (end 136.85 119.8) (width 0.22) (layer "F.Cu") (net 13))
 (segment (start 136.9 117.3) (end 136.85 117.35) (width 0.22) (layer "F.Cu") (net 13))
 (segment (start 136.85 119.8) (end 136 120.65) (width 0.22) (layer "F.Cu") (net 13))
 (via (at 136.9 117.3) (size 0.6) (drill 0.3) (layers "F.Cu" "B.Cu") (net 13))
 (via (at 136 120.65) (size 0.6) (drill 0.3) (layers "F.Cu" "B.Cu") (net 13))
 (segment (start 135.4 117.05) (end 135.7 116.75) (width 0.22) (layer "B.Cu") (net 13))
 (segment (start 135.7 116.75) (end 136.35 116.75) (width 0.22) (layer "B.Cu") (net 13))
 (segment (start 135.35 121.3) (end 133.65 121.3) (width 0.22) (layer "B.Cu") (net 13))
 (segment (start 136 120.65) (end 135.35 121.3) (width 0.22) (layer "B.Cu") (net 13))
 (segment (start 135.4 117.45) (end 135.4 117.05) (width 0.22) (layer "B.Cu") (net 13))
 (segment (start 136.35 116.75) (end 136.9 117.3) (width 0.22) (layer "B.Cu") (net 13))
 (segment (start 132.95 120.680978) (end 133.330978 120.3) (width 0.22) (layer "B.Cu") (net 12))
 (segment (start 136.675 122.7) (end 136.675 120.375) (width 0.22) (layer "B.Cu") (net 12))
 (segment (start 135.35 120) (end 135.65 120) (width 0.22) (layer "B.Cu") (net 12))
 (segment (start 132.95 121.3) (end 132.95 120.680978) (width 0.22) (layer "B.Cu") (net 12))
 (segment (start 136.675 120.375) (end 136.3 120) (width 0.22) (layer "B.Cu") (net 12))
 (segment (start 135.05 120.3) (end 135.35 120) (width 0.22) (layer "B.Cu") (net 12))
 (segment (start 135.4 120) (end 135.4 119.05) (width 0.22) (layer "B.Cu") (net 12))
 (segment (start 133.330978 120.3) (end 135.05 120.3) (width 0.22) (layer "B.Cu") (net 12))
 (segment (start 136.3 120) (end 135.65 120) (width 0.22) (layer "B.Cu") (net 12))
 (segment (start 130.75 123.5) (end 130.130978 123.5) (width 0.22) (layer "B.Cu") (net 20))
 (segment (start 129.95 124.55) (end 130.3 124.9) (width 0.22) (layer "B.Cu") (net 20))
 (segment (start 130.3 124.9) (end 131.2 124.9) (width 0.22) (layer "B.Cu") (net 20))
 (segment (start 131.45 124.65) (end 131.45 124.2) (width 0.22) (layer "B.Cu") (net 20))
 (segment (start 131.2 124.9) (end 131.45 124.65) (width 0.22) (layer "B.Cu") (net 20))
 (segment (start 129.95 123.680978) (end 129.95 124.55) (width 0.22) (layer "B.Cu") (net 20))
 (segment (start 130.130978 123.5) (end 129.95 123.680978) (width 0.22) (layer "B.Cu") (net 20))
 (segment (start 127.525 121) (end 125.975 122.55) (width 0.3) (layer "B.Cu") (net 10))
 (segment (start 123.2 124.8) (end 124.55 124.8) (width 0.3) (layer "B.Cu") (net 10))
 (segment (start 128.625 122) (end 127.625 121) (width 0.3) (layer "B.Cu") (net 10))
 (segment (start 127.625 121) (end 127.525 121) (width 0.3) (layer "B.Cu") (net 10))
 (segment (start 127.625 120.975) (end 126.85 120.2) (width 0.3) (layer "B.Cu") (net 10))
 (segment (start 127.625 121) (end 127.625 120.975) (width 0.3) (layer "B.Cu") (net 10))
 (segment (start 125.975 123.375) (end 125.975 122.55) (width 0.3) (layer "B.Cu") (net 10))
 (segment (start 130.75 122) (end 128.625 122) (width 0.3) (layer "B.Cu") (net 10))
 (segment (start 126.85 120.2) (end 126.85 119.5) (width 0.3) (layer "B.Cu") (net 10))
 (segment (start 124.55 124.8) (end 125.975 123.375) (width 0.3) (layer "B.Cu") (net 10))
 (segment (start 128.8 118.55) (end 128.725 118.55) (width 0.6) (layer "B.Cu") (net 1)))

